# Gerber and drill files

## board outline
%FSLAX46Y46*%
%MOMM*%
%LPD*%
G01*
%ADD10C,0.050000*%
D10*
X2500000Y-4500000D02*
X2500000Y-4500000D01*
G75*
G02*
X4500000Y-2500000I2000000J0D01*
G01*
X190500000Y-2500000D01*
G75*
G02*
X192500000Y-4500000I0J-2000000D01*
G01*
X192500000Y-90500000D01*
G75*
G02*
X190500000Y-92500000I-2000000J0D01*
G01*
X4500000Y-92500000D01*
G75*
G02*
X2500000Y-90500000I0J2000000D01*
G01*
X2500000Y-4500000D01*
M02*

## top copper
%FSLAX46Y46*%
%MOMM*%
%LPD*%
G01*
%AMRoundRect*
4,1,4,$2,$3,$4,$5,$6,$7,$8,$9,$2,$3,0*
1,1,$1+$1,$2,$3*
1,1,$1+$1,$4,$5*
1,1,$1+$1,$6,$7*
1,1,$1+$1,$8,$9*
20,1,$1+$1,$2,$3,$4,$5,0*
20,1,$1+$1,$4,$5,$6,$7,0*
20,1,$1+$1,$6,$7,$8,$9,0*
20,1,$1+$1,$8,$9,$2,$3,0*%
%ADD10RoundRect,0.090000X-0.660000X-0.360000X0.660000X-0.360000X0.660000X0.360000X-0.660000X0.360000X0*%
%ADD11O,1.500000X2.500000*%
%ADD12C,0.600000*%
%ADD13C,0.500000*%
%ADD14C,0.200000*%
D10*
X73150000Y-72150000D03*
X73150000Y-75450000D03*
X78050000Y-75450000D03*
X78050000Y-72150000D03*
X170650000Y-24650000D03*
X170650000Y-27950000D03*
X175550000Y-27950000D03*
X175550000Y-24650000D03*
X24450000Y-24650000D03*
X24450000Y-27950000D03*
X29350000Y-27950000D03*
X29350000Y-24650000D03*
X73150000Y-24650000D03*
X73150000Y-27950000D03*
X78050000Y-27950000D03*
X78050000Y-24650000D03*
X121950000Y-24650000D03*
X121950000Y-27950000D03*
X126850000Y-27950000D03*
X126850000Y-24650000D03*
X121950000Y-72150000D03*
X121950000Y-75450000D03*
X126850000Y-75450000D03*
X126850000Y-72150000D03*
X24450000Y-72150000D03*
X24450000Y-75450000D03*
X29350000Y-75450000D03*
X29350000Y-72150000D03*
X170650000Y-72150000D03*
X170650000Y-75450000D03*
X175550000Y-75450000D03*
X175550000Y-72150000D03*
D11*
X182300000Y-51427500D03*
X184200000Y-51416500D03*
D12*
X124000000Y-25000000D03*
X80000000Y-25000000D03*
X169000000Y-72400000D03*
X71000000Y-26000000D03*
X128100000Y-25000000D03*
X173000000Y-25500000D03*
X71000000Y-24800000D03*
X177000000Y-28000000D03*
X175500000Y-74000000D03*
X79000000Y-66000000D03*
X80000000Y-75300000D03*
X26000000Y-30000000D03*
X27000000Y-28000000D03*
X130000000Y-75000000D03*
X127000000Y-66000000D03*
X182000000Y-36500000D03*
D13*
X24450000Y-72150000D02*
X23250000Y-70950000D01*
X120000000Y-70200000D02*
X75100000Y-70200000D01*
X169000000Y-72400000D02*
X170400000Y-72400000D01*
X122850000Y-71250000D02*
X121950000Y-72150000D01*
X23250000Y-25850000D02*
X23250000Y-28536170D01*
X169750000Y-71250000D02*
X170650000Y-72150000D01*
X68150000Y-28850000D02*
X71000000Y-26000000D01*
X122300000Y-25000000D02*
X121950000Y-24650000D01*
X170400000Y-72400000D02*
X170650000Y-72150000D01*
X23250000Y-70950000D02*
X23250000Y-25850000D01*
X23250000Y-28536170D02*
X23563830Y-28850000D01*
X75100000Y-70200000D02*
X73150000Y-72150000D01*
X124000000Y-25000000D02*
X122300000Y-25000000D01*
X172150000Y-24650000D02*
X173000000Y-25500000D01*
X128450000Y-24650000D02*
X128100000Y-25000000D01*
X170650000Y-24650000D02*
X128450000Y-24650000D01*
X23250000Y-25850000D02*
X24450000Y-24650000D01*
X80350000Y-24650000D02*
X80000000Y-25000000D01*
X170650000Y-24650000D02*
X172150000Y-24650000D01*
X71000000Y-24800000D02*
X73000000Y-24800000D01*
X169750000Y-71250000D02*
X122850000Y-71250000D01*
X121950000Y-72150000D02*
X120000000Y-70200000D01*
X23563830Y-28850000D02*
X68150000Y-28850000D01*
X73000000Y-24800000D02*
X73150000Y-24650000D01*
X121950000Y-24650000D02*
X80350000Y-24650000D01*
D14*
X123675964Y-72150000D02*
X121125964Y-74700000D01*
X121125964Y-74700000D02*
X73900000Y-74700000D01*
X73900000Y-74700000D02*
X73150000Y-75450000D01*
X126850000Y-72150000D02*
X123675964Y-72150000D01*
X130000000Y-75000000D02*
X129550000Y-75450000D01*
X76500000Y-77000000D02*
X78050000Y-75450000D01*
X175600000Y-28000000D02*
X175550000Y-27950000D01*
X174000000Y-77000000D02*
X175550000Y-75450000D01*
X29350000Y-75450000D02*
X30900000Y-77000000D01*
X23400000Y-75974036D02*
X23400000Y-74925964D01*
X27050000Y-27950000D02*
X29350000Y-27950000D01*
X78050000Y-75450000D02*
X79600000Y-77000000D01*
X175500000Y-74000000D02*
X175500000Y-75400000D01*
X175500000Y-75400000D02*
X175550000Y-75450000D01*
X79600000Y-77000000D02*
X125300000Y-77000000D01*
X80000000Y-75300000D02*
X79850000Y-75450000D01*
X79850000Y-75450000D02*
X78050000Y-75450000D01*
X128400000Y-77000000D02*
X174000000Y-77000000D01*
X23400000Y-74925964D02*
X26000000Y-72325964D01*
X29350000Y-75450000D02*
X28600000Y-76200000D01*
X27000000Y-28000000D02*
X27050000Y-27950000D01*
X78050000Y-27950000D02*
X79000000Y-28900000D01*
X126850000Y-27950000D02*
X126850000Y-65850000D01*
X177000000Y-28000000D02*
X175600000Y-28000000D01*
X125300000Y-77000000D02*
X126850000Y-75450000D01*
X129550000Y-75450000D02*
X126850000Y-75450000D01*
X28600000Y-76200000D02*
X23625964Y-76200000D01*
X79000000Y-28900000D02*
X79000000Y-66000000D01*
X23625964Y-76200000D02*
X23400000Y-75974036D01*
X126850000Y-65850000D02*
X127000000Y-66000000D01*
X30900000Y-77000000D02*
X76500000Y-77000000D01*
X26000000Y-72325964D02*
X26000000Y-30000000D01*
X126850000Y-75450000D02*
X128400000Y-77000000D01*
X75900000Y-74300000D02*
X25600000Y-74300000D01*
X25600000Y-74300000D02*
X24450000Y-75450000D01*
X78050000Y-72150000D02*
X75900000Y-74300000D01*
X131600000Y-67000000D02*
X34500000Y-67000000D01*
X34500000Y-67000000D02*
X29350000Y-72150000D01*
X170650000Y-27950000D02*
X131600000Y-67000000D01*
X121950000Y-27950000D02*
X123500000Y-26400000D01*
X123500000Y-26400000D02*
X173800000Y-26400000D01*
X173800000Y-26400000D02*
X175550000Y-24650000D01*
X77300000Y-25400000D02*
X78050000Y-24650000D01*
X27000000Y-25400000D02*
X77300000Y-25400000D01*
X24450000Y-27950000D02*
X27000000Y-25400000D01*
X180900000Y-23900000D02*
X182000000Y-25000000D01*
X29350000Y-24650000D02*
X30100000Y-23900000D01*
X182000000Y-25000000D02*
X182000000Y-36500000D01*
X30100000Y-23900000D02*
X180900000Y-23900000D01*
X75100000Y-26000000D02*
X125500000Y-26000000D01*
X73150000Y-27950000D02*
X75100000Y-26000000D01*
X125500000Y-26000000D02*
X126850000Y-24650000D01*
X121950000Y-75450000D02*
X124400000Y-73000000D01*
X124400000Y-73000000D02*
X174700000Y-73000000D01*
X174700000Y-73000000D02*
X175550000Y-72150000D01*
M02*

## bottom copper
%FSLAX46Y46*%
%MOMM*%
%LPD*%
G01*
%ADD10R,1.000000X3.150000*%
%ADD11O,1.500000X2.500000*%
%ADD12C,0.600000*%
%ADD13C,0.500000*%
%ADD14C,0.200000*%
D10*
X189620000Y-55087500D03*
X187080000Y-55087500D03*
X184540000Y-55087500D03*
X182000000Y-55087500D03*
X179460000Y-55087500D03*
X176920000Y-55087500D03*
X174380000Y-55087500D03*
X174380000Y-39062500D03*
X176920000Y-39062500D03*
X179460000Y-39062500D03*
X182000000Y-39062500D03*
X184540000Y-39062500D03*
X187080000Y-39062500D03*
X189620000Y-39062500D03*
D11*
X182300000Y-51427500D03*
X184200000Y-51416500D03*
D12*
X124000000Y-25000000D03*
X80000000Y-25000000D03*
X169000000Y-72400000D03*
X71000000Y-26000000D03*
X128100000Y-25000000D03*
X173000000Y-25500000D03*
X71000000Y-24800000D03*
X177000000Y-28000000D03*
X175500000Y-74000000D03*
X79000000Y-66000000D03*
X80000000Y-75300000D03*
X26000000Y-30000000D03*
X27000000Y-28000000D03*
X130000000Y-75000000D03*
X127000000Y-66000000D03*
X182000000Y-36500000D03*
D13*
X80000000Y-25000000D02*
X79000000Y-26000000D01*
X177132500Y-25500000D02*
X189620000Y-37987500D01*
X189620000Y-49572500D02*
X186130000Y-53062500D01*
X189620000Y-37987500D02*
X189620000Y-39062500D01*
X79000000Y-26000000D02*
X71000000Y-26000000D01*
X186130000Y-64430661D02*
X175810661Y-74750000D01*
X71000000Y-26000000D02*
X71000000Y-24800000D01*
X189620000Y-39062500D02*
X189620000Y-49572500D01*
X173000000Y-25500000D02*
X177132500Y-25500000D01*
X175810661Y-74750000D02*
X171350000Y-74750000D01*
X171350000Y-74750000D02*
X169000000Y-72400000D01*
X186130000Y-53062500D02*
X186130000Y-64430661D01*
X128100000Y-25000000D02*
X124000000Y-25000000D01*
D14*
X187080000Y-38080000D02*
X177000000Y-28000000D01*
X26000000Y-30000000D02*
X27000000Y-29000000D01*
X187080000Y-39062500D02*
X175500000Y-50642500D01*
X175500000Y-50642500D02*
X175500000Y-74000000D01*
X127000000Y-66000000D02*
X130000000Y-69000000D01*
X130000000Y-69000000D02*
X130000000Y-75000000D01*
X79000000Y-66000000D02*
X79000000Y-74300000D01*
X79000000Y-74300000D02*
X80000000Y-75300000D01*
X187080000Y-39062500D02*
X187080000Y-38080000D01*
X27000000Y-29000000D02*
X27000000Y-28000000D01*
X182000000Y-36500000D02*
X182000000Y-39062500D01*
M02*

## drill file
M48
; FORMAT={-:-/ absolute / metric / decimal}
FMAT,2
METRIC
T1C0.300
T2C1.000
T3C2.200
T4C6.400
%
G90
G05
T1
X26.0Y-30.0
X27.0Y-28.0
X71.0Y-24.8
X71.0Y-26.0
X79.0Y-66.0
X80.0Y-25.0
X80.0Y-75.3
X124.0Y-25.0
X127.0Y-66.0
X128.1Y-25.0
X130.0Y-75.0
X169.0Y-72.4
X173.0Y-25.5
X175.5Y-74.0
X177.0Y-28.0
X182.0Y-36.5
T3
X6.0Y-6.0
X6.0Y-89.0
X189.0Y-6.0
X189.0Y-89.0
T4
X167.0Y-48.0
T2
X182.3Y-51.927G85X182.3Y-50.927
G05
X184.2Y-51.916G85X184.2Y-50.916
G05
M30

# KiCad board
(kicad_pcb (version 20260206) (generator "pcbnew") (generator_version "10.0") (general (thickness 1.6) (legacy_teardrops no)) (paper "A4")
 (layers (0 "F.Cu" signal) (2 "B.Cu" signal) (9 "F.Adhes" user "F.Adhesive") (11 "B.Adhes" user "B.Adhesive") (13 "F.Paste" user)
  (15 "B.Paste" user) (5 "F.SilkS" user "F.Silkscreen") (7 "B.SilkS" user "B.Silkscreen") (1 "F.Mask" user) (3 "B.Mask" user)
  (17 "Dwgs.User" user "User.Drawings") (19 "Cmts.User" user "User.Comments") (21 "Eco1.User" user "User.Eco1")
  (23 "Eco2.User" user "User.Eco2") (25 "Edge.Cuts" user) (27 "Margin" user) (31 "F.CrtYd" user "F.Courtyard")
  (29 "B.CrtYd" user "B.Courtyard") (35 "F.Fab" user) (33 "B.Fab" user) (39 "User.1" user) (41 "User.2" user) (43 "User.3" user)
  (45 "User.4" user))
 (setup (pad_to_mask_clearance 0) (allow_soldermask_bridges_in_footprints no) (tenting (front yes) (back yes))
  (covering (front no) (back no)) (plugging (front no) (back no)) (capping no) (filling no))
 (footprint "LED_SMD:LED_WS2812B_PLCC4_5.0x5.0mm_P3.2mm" (layer "F.Cu") (at 75.6 73.8)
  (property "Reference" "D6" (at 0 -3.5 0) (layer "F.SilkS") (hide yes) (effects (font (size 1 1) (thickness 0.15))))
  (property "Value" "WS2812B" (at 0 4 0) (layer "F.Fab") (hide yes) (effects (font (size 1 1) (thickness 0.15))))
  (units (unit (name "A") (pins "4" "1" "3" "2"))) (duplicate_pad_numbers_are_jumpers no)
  (pad "1" smd roundrect (at -2.45 -1.65) (size 1.5 0.9) (layers "F.Cu" "F.Mask" "F.Paste") (roundrect_rratio 0.1) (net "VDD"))
  (pad "2" smd roundrect (at -2.45 1.65) (size 1.5 0.9) (layers "F.Cu" "F.Mask" "F.Paste") (roundrect_rratio 0.1) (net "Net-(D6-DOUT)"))
  (pad "3" smd roundrect (at 2.45 1.65) (size 1.5 0.9) (layers "F.Cu" "F.Mask" "F.Paste") (roundrect_rratio 0.1) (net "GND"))
  (pad "4" smd roundrect (at 2.45 -1.65) (size 1.5 0.9) (layers "F.Cu" "F.Mask" "F.Paste") (roundrect_rratio 0.1) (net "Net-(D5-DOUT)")))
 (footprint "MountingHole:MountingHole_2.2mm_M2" (layer "F.Cu") (at 189 89)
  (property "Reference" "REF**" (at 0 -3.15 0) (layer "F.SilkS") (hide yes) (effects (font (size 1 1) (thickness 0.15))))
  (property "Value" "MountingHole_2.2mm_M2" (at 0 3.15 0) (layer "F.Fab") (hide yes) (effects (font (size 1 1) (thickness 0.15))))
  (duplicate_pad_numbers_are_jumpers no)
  (pad "" np_thru_hole circle (at 0 0) (size 2.2 2.2) (drill 2.2) (layers "*.Cu" "*.Mask")))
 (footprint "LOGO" (layer "F.Cu") (at 99 42)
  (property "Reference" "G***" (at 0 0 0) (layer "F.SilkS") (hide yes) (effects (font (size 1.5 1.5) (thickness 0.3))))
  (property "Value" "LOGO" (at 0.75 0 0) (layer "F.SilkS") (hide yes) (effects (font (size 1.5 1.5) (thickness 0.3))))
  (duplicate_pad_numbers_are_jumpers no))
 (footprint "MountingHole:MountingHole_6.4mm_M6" (layer "F.Cu") (at 167 48)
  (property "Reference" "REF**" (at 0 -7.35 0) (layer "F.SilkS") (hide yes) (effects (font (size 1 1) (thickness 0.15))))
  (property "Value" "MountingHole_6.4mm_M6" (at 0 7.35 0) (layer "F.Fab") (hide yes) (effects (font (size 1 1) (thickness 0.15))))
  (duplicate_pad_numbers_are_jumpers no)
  (pad "" np_thru_hole circle (at 0 0) (size 6.4 6.4) (drill 6.4) (layers "*.Cu" "*.Mask")))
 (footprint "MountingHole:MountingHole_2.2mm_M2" (layer "F.Cu") (at 6 6)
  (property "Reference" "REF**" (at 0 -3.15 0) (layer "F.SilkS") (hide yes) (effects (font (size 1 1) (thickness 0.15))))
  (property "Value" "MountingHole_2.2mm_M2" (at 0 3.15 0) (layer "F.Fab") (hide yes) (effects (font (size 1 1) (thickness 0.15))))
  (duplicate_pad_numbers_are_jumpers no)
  (pad "" np_thru_hole circle (at 0 0) (size 2.2 2.2) (drill 2.2) (layers "*.Cu" "*.Mask")))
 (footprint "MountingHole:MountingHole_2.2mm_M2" (layer "F.Cu") (at 189 6)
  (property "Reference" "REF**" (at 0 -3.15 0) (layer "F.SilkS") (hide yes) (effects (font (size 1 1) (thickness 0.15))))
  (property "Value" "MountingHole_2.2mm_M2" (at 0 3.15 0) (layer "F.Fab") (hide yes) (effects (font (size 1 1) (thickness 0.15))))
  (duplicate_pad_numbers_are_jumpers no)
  (pad "" np_thru_hole circle (at 0 0) (size 2.2 2.2) (drill 2.2) (layers "*.Cu" "*.Mask")))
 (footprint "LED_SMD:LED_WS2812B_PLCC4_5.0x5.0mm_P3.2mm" (layer "F.Cu") (at 173.1 26.3)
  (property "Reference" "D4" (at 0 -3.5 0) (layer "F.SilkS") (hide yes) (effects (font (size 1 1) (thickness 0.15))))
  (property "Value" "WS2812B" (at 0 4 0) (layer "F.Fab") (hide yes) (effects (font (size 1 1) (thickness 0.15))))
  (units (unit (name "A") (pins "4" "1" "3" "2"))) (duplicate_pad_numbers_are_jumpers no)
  (pad "1" smd roundrect (at -2.45 -1.65) (size 1.5 0.9) (layers "F.Cu" "F.Mask" "F.Paste") (roundrect_rratio 0.1) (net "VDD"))
  (pad "2" smd roundrect (at -2.45 1.65) (size 1.5 0.9) (layers "F.Cu" "F.Mask" "F.Paste") (roundrect_rratio 0.1) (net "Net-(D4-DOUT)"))
  (pad "3" smd roundrect (at 2.45 1.65) (size 1.5 0.9) (layers "F.Cu" "F.Mask" "F.Paste") (roundrect_rratio 0.1) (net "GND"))
  (pad "4" smd roundrect (at 2.45 -1.65) (size 1.5 0.9) (layers "F.Cu" "F.Mask" "F.Paste") (roundrect_rratio 0.1) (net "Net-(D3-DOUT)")))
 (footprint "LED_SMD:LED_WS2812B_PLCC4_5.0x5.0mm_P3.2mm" (layer "F.Cu") (at 26.9 26.3)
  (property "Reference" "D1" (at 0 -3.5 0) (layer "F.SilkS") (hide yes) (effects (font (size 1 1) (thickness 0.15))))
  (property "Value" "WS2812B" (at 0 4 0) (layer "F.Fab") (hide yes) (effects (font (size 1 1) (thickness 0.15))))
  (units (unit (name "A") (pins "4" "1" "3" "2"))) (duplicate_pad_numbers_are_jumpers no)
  (pad "1" smd roundrect (at -2.45 -1.65) (size 1.5 0.9) (layers "F.Cu" "F.Mask" "F.Paste") (roundrect_rratio 0.1) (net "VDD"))
  (pad "2" smd roundrect (at -2.45 1.65) (size 1.5 0.9) (layers "F.Cu" "F.Mask" "F.Paste") (roundrect_rratio 0.1) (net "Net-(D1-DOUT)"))
  (pad "3" smd roundrect (at 2.45 1.65) (size 1.5 0.9) (layers "F.Cu" "F.Mask" "F.Paste") (roundrect_rratio 0.1) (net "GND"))
  (pad "4" smd roundrect (at 2.45 -1.65) (size 1.5 0.9) (layers "F.Cu" "F.Mask" "F.Paste") (roundrect_rratio 0.1) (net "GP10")))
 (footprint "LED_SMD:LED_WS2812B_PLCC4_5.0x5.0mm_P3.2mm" (layer "F.Cu") (at 75.6 26.3)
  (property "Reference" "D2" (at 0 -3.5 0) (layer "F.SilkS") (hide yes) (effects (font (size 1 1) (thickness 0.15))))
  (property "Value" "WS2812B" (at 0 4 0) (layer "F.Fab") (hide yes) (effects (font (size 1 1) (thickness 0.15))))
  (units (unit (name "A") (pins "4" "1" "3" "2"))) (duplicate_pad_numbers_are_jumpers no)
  (pad "1" smd roundrect (at -2.45 -1.65) (size 1.5 0.9) (layers "F.Cu" "F.Mask" "F.Paste") (roundrect_rratio 0.1) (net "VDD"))
  (pad "2" smd roundrect (at -2.45 1.65) (size 1.5 0.9) (layers "F.Cu" "F.Mask" "F.Paste") (roundrect_rratio 0.1) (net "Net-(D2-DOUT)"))
  (pad "3" smd roundrect (at 2.45 1.65) (size 1.5 0.9) (layers "F.Cu" "F.Mask" "F.Paste") (roundrect_rratio 0.1) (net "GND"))
  (pad "4" smd roundrect (at 2.45 -1.65) (size 1.5 0.9) (layers "F.Cu" "F.Mask" "F.Paste") (roundrect_rratio 0.1) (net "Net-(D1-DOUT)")))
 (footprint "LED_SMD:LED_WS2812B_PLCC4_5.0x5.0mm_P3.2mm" (layer "F.Cu") (at 124.4 26.3)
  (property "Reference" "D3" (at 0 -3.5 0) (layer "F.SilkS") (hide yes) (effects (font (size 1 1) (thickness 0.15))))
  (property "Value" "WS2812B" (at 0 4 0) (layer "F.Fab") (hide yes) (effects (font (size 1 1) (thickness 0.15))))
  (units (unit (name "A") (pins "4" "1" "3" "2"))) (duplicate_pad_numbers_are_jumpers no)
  (pad "1" smd roundrect (at -2.45 -1.65) (size 1.5 0.9) (layers "F.Cu" "F.Mask" "F.Paste") (roundrect_rratio 0.1) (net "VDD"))
  (pad "2" smd roundrect (at -2.45 1.65) (size 1.5 0.9) (layers "F.Cu" "F.Mask" "F.Paste") (roundrect_rratio 0.1) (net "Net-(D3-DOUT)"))
  (pad "3" smd roundrect (at 2.45 1.65) (size 1.5 0.9) (layers "F.Cu" "F.Mask" "F.Paste") (roundrect_rratio 0.1) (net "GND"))
  (pad "4" smd roundrect (at 2.45 -1.65) (size 1.5 0.9) (layers "F.Cu" "F.Mask" "F.Paste") (roundrect_rratio 0.1) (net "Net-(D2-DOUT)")))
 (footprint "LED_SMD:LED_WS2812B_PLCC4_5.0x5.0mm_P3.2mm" (layer "F.Cu") (at 124.4 73.8)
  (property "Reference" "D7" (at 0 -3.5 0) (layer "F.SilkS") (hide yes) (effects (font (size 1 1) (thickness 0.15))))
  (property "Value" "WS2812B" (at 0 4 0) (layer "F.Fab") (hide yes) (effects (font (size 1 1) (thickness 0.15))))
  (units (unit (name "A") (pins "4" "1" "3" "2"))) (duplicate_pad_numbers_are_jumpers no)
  (pad "1" smd roundrect (at -2.45 -1.65) (size 1.5 0.9) (layers "F.Cu" "F.Mask" "F.Paste") (roundrect_rratio 0.1) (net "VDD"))
  (pad "2" smd roundrect (at -2.45 1.65) (size 1.5 0.9) (layers "F.Cu" "F.Mask" "F.Paste") (roundrect_rratio 0.1) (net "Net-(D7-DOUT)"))
  (pad "3" smd roundrect (at 2.45 1.65) (size 1.5 0.9) (layers "F.Cu" "F.Mask" "F.Paste") (roundrect_rratio 0.1) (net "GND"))
  (pad "4" smd roundrect (at 2.45 -1.65) (size 1.5 0.9) (layers "F.Cu" "F.Mask" "F.Paste") (roundrect_rratio 0.1) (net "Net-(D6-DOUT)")))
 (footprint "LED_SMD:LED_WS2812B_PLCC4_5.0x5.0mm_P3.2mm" (layer "F.Cu") (at 26.9 73.8)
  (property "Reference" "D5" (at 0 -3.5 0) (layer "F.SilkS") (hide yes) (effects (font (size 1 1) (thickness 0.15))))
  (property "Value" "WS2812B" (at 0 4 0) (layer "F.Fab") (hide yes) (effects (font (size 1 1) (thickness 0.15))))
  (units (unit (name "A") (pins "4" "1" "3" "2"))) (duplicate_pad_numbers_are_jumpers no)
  (pad "1" smd roundrect (at -2.45 -1.65) (size 1.5 0.9) (layers "F.Cu" "F.Mask" "F.Paste") (roundrect_rratio 0.1) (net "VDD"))
  (pad "2" smd roundrect (at -2.45 1.65) (size 1.5 0.9) (layers "F.Cu" "F.Mask" "F.Paste") (roundrect_rratio 0.1) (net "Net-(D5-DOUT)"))
  (pad "3" smd roundrect (at 2.45 1.65) (size 1.5 0.9) (layers "F.Cu" "F.Mask" "F.Paste") (roundrect_rratio 0.1) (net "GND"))
  (pad "4" smd roundrect (at 2.45 -1.65) (size 1.5 0.9) (layers "F.Cu" "F.Mask" "F.Paste") (roundrect_rratio 0.1) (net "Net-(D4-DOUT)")))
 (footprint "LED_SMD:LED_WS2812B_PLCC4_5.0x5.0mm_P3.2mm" (layer "F.Cu") (at 173.1 73.8)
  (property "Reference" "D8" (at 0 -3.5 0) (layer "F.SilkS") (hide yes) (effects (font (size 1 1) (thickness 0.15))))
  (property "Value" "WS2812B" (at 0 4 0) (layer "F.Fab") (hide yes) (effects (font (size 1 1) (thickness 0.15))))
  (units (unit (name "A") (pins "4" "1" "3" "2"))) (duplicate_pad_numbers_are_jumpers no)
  (pad "1" smd roundrect (at -2.45 -1.65) (size 1.5 0.9) (layers "F.Cu" "F.Mask" "F.Paste") (roundrect_rratio 0.1) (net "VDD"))
  (pad "2" smd roundrect (at -2.45 1.65) (size 1.5 0.9) (layers "F.Cu" "F.Mask" "F.Paste") (roundrect_rratio 0.1)
   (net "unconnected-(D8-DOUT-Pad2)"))
  (pad "3" smd roundrect (at 2.45 1.65) (size 1.5 0.9) (layers "F.Cu" "F.Mask" "F.Paste") (roundrect_rratio 0.1) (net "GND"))
  (pad "4" smd roundrect (at 2.45 -1.65) (size 1.5 0.9) (layers "F.Cu" "F.Mask" "F.Paste") (roundrect_rratio 0.1) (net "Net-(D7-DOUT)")))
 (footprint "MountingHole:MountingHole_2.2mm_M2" (layer "F.Cu") (at 6 89)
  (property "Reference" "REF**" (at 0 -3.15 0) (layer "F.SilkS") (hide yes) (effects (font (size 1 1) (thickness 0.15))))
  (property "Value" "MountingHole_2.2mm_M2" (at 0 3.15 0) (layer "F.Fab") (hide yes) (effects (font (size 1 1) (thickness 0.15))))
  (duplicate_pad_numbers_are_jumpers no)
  (pad "" np_thru_hole circle (at 0 0) (size 2.2 2.2) (drill 2.2) (layers "*.Cu" "*.Mask")))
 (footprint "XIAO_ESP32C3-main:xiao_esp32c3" (layer "B.Cu") (at 180.2 46.4875 90)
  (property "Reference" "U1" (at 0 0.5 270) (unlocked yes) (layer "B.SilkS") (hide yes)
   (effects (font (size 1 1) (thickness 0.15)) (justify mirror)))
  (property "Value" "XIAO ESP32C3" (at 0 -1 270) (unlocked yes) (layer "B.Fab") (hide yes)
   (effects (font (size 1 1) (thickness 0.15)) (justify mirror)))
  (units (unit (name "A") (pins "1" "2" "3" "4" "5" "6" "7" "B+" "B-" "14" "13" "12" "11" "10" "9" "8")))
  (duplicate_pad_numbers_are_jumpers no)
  (pad "1" smd rect (at -8.6 9.42 90) (size 3.15 1) (layers "B.Cu" "B.Mask" "B.Paste") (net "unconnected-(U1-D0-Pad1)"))
  (pad "2" smd rect (at -8.6 6.88 90) (size 3.15 1) (layers "B.Cu" "B.Mask" "B.Paste") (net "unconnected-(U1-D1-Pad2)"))
  (pad "3" smd rect (at -8.6 4.34 90) (size 3.15 1) (layers "B.Cu" "B.Mask" "B.Paste") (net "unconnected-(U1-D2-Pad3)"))
  (pad "4" smd rect (at -8.6 1.8 90) (size 3.15 1) (layers "B.Cu" "B.Mask" "B.Paste") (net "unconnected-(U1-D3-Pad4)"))
  (pad "5" smd rect (at -8.6 -0.74 90) (size 3.15 1) (layers "B.Cu" "B.Mask" "B.Paste") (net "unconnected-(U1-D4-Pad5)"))
  (pad "6" smd rect (at -8.6 -3.28 90) (size 3.15 1) (layers "B.Cu" "B.Mask" "B.Paste") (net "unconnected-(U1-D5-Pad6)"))
  (pad "7" smd rect (at -8.6 -5.82 90) (size 3.15 1) (layers "B.Cu" "B.Mask" "B.Paste") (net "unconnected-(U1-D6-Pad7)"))
  (pad "8" smd rect (at 7.425 -5.82 90) (size 3.15 1) (layers "B.Cu" "B.Mask" "B.Paste") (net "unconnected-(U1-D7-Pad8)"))
  (pad "9" smd rect (at 7.425 -3.28 90) (size 3.15 1) (layers "B.Cu" "B.Mask" "B.Paste") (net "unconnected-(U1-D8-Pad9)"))
  (pad "10" smd rect (at 7.425 -0.74 90) (size 3.15 1) (layers "B.Cu" "B.Mask" "B.Paste") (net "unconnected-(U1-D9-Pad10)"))
  (pad "11" smd rect (at 7.425 1.8 90) (size 3.15 1) (layers "B.Cu" "B.Mask" "B.Paste") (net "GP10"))
  (pad "12" smd rect (at 7.425 4.34 90) (size 3.15 1) (layers "B.Cu" "B.Mask" "B.Paste") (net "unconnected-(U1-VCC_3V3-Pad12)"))
  (pad "13" smd rect (at 7.425 6.88 90) (size 3.15 1) (layers "B.Cu" "B.Mask" "B.Paste") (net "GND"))
  (pad "14" smd rect (at 7.425 9.42 90) (size 3.15 1) (layers "B.Cu" "B.Mask" "B.Paste") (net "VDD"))
  (pad "B+" thru_hole oval (at -4.94 2.1 90) (size 2.5 1.5) (drill oval 2 1) (layers "*.Cu" "*.Mask") (remove_unused_layers no)
   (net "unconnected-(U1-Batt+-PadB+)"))
  (pad "B-" thru_hole oval (at -4.929 4 90) (size 2.5 1.5) (drill oval 2 1) (layers "*.Cu" "*.Mask") (remove_unused_layers no)
   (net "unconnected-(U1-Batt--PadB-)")))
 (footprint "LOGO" (layer "B.Cu") (at 100 42 180)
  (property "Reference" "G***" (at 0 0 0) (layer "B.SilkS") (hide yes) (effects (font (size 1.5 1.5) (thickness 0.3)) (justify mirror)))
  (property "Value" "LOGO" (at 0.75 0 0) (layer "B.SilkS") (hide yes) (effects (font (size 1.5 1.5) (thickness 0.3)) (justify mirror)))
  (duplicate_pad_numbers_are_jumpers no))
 (gr_rect (start 2.5 2.5) (end 192.5 92.5) (radius 2) (stroke (width 0.05) (type solid)) (fill no) (layer "Edge.Cuts"))
 (segment (start 24.45 72.15) (end 23.25 70.95) (width 0.5) (layer "F.Cu") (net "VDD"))
 (segment (start 120 70.2) (end 75.1 70.2) (width 0.5) (layer "F.Cu") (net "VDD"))
 (segment (start 169 72.4) (end 170.4 72.4) (width 0.5) (layer "F.Cu") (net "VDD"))
 (segment (start 122.85 71.25) (end 121.95 72.15) (width 0.5) (layer "F.Cu") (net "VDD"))
 (segment (start 23.25 25.85) (end 23.25 28.53617) (width 0.5) (layer "F.Cu") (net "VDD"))
 (segment (start 169.75 71.25) (end 170.65 72.15) (width 0.5) (layer "F.Cu") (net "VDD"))
 (segment (start 68.15 28.85) (end 71 26) (width 0.5) (layer "F.Cu") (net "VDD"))
 (segment (start 122.3 25) (end 121.95 24.65) (width 0.5) (layer "F.Cu") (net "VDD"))
 (segment (start 170.4 72.4) (end 170.65 72.15) (width 0.5) (layer "F.Cu") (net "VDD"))
 (segment (start 23.25 70.95) (end 23.25 25.85) (width 0.5) (layer "F.Cu") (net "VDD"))
 (segment (start 23.25 28.53617) (end 23.56383 28.85) (width 0.5) (layer "F.Cu") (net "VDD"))
 (segment (start 75.1 70.2) (end 73.15 72.15) (width 0.5) (layer "F.Cu") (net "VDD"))
 (segment (start 124 25) (end 122.3 25) (width 0.5) (layer "F.Cu") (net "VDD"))
 (segment (start 172.15 24.65) (end 173 25.5) (width 0.5) (layer "F.Cu") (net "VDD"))
 (segment (start 128.45 24.65) (end 128.1 25) (width 0.5) (layer "F.Cu") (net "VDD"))
 (segment (start 170.65 24.65) (end 128.45 24.65) (width 0.5) (layer "F.Cu") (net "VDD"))
 (segment (start 23.25 25.85) (end 24.45 24.65) (width 0.5) (layer "F.Cu") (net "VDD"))
 (segment (start 80.35 24.65) (end 80 25) (width 0.5) (layer "F.Cu") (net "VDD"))
 (segment (start 170.65 24.65) (end 172.15 24.65) (width 0.5) (layer "F.Cu") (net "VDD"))
 (segment (start 71 24.8) (end 73 24.8) (width 0.5) (layer "F.Cu") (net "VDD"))
 (segment (start 169.75 71.25) (end 122.85 71.25) (width 0.5) (layer "F.Cu") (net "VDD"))
 (segment (start 121.95 72.15) (end 120 70.2) (width 0.5) (layer "F.Cu") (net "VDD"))
 (segment (start 23.56383 28.85) (end 68.15 28.85) (width 0.5) (layer "F.Cu") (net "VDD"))
 (segment (start 73 24.8) (end 73.15 24.65) (width 0.5) (layer "F.Cu") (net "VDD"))
 (segment (start 121.95 24.65) (end 80.35 24.65) (width 0.5) (layer "F.Cu") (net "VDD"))
 (via (at 124 25) (size 0.6) (drill 0.3) (layers "F.Cu" "B.Cu") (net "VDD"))
 (via (at 80 25) (size 0.6) (drill 0.3) (layers "F.Cu" "B.Cu") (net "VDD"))
 (via (at 169 72.4) (size 0.6) (drill 0.3) (layers "F.Cu" "B.Cu") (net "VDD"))
 (via (at 71 26) (size 0.6) (drill 0.3) (layers "F.Cu" "B.Cu") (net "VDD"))
 (via (at 128.1 25) (size 0.6) (drill 0.3) (layers "F.Cu" "B.Cu") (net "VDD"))
 (via (at 173 25.5) (size 0.6) (drill 0.3) (layers "F.Cu" "B.Cu") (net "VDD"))
 (via (at 71 24.8) (size 0.6) (drill 0.3) (layers "F.Cu" "B.Cu") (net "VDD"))
 (segment (start 80 25) (end 79 26) (width 0.5) (layer "B.Cu") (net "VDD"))
 (segment (start 177.1325 25.5) (end 189.62 37.9875) (width 0.5) (layer "B.Cu") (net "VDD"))
 (segment (start 189.62 49.5725) (end 186.13 53.0625) (width 0.5) (layer "B.Cu") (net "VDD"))
 (segment (start 189.62 37.9875) (end 189.62 39.0625) (width 0.5) (layer "B.Cu") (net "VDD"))
 (segment (start 79 26) (end 71 26) (width 0.5) (layer "B.Cu") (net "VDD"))
 (segment (start 186.13 64.430661) (end 175.810661 74.75) (width 0.5) (layer "B.Cu") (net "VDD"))
 (segment (start 71 26) (end 71 24.8) (width 0.5) (layer "B.Cu") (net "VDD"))
 (segment (start 189.62 39.0625) (end 189.62 49.5725) (width 0.5) (layer "B.Cu") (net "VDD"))
 (segment (start 173 25.5) (end 177.1325 25.5) (width 0.5) (layer "B.Cu") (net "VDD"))
 (segment (start 175.810661 74.75) (end 171.35 74.75) (width 0.5) (layer "B.Cu") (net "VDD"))
 (segment (start 171.35 74.75) (end 169 72.4) (width 0.5) (layer "B.Cu") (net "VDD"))
 (segment (start 186.13 53.0625) (end 186.13 64.430661) (width 0.5) (layer "B.Cu") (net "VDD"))
 (segment (start 128.1 25) (end 124 25) (width 0.5) (layer "B.Cu") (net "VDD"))
 (segment (start 123.675964 72.15) (end 121.125964 74.7) (width 0.2) (layer "F.Cu") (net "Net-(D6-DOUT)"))
 (segment (start 121.125964 74.7) (end 73.9 74.7) (width 0.2) (layer "F.Cu") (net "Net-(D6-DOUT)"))
 (segment (start 73.9 74.7) (end 73.15 75.45) (width 0.2) (layer "F.Cu") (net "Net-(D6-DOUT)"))
 (segment (start 126.85 72.15) (end 123.675964 72.15) (width 0.2) (layer "F.Cu") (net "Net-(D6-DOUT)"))
 (segment (start 130 75) (end 129.55 75.45) (width 0.2) (layer "F.Cu") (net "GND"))
 (segment (start 76.5 77) (end 78.05 75.45) (width 0.2) (layer "F.Cu") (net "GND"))
 (segment (start 175.6 28) (end 175.55 27.95) (width 0.2) (layer "F.Cu") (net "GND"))
 (segment (start 174 77) (end 175.55 75.45) (width 0.2) (layer "F.Cu") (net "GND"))
 (segment (start 29.35 75.45) (end 30.9 77) (width 0.2) (layer "F.Cu") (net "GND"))
 (segment (start 23.4 75.974036) (end 23.4 74.925964) (width 0.2) (layer "F.Cu") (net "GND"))
 (segment (start 27.05 27.95) (end 29.35 27.95) (width 0.2) (layer "F.Cu") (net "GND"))
 (segment (start 78.05 75.45) (end 79.6 77) (width 0.2) (layer "F.Cu") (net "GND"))
 (segment (start 175.5 74) (end 175.5 75.4) (width 0.2) (layer "F.Cu") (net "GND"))
 (segment (start 175.5 75.4) (end 175.55 75.45) (width 0.2) (layer "F.Cu") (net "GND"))
 (segment (start 79.6 77) (end 125.3 77) (width 0.2) (layer "F.Cu") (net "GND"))
 (segment (start 80 75.3) (end 79.85 75.45) (width 0.2) (layer "F.Cu") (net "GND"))
 (segment (start 79.85 75.45) (end 78.05 75.45) (width 0.2) (layer "F.Cu") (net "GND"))
 (segment (start 128.4 77) (end 174 77) (width 0.2) (layer "F.Cu") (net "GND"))
 (segment (start 23.4 74.925964) (end 26 72.325964) (width 0.2) (layer "F.Cu") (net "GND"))
 (segment (start 29.35 75.45) (end 28.6 76.2) (width 0.2) (layer "F.Cu") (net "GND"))
 (segment (start 27 28) (end 27.05 27.95) (width 0.2) (layer "F.Cu") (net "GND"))
 (segment (start 78.05 27.95) (end 79 28.9) (width 0.2) (layer "F.Cu") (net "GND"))
 (segment (start 126.85 27.95) (end 126.85 65.85) (width 0.2) (layer "F.Cu") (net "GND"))
 (segment (start 177 28) (end 175.6 28) (width 0.2) (layer "F.Cu") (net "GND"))
 (segment (start 125.3 77) (end 126.85 75.45) (width 0.2) (layer "F.Cu") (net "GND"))
 (segment (start 129.55 75.45) (end 126.85 75.45) (width 0.2) (layer "F.Cu") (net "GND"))
 (segment (start 28.6 76.2) (end 23.625964 76.2) (width 0.2) (layer "F.Cu") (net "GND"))
 (segment (start 79 28.9) (end 79 66) (width 0.2) (layer "F.Cu") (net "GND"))
 (segment (start 23.625964 76.2) (end 23.4 75.974036) (width 0.2) (layer "F.Cu") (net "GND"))
 (segment (start 126.85 65.85) (end 127 66) (width 0.2) (layer "F.Cu") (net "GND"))
 (segment (start 30.9 77) (end 76.5 77) (width 0.2) (layer "F.Cu") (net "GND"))
 (segment (start 26 72.325964) (end 26 30) (width 0.2) (layer "F.Cu") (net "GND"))
 (segment (start 126.85 75.45) (end 128.4 77) (width 0.2) (layer "F.Cu") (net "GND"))
 (via (at 177 28) (size 0.6) (drill 0.3) (layers "F.Cu" "B.Cu") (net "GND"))
 (via (at 175.5 74) (size 0.6) (drill 0.3) (layers "F.Cu" "B.Cu") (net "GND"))
 (via (at 79 66) (size 0.6) (drill 0.3) (layers "F.Cu" "B.Cu") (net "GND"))
 (via (at 80 75.3) (size 0.6) (drill 0.3) (layers "F.Cu" "B.Cu") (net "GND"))
 (via (at 26 30) (size 0.6) (drill 0.3) (layers "F.Cu" "B.Cu") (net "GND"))
 (via (at 27 28) (size 0.6) (drill 0.3) (layers "F.Cu" "B.Cu") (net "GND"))
 (via (at 130 75) (size 0.6) (drill 0.3) (layers "F.Cu" "B.Cu") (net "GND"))
 (via (at 127 66) (size 0.6) (drill 0.3) (layers "F.Cu" "B.Cu") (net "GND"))
 (segment (start 187.08 38.08) (end 177 28) (width 0.2) (layer "B.Cu") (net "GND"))
 (segment (start 26 30) (end 27 29) (width 0.2) (layer "B.Cu") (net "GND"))
 (segment (start 187.08 39.0625) (end 175.5 50.6425) (width 0.2) (layer "B.Cu") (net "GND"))
 (segment (start 175.5 50.6425) (end 175.5 74) (width 0.2) (layer "B.Cu") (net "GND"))
 (segment (start 127 66) (end 130 69) (width 0.2) (layer "B.Cu") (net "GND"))
 (segment (start 130 69) (end 130 75) (width 0.2) (layer "B.Cu") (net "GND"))
 (segment (start 79 66) (end 79 74.3) (width 0.2) (layer "B.Cu") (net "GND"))
 (segment (start 79 74.3) (end 80 75.3) (width 0.2) (layer "B.Cu") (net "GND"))
 (segment (start 187.08 39.0625) (end 187.08 38.08) (width 0.2) (layer "B.Cu") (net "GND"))
 (segment (start 27 29) (end 27 28) (width 0.2) (layer "B.Cu") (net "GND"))
 (segment (start 75.9 74.3) (end 25.6 74.3) (width 0.2) (layer "F.Cu") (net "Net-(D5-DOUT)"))
 (segment (start 25.6 74.3) (end 24.45 75.45) (width 0.2) (layer "F.Cu") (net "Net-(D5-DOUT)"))
 (segment (start 78.05 72.15) (end 75.9 74.3) (width 0.2) (layer "F.Cu") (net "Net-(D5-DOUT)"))
 (segment (start 131.6 67) (end 34.5 67) (width 0.2) (layer "F.Cu") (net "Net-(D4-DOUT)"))
 (segment (start 34.5 67) (end 29.35 72.15) (width 0.2) (layer "F.Cu") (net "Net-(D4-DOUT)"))
 (segment (start 170.65 27.95) (end 131.6 67) (width 0.2) (layer "F.Cu") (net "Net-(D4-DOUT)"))
 (segment (start 121.95 27.95) (end 123.5 26.4) (width 0.2) (layer "F.Cu") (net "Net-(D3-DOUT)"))
 (segment (start 123.5 26.4) (end 173.8 26.4) (width 0.2) (layer "F.Cu") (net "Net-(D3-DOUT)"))
 (segment (start 173.8 26.4) (end 175.55 24.65) (width 0.2) (layer "F.Cu") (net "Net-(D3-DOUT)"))
 (segment (start 77.3 25.4) (end 78.05 24.65) (width 0.2) (layer "F.Cu") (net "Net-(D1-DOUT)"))
 (segment (start 27 25.4) (end 77.3 25.4) (width 0.2) (layer "F.Cu") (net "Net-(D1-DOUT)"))
 (segment (start 24.45 27.95) (end 27 25.4) (width 0.2) (layer "F.Cu") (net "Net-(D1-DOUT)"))
 (segment (start 180.9 23.9) (end 182 25) (width 0.2) (layer "F.Cu") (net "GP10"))
 (segment (start 29.35 24.65) (end 30.1 23.9) (width 0.2) (layer "F.Cu") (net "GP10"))
 (segment (start 182 25) (end 182 36.5) (width 0.2) (layer "F.Cu") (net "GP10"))
 (segment (start 30.1 23.9) (end 180.9 23.9) (width 0.2) (layer "F.Cu") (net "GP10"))
 (via (at 182 36.5) (size 0.6) (drill 0.3) (layers "F.Cu" "B.Cu") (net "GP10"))
 (segment (start 182 36.5) (end 182 39.0625) (width 0.2) (layer "B.Cu") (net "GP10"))
 (segment (start 75.1 26) (end 125.5 26) (width 0.2) (layer "F.Cu") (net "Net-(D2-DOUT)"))
 (segment (start 73.15 27.95) (end 75.1 26) (width 0.2) (layer "F.Cu") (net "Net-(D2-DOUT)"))
 (segment (start 125.5 26) (end 126.85 24.65) (width 0.2) (layer "F.Cu") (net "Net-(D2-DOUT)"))
 (segment (start 121.95 75.45) (end 124.4 73) (width 0.2) (layer "F.Cu") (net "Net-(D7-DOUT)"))
 (segment (start 124.4 73) (end 174.7 73) (width 0.2) (layer "F.Cu") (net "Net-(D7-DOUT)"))
 (segment (start 174.7 73) (end 175.55 72.15) (width 0.2) (layer "F.Cu") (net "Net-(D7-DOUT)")))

